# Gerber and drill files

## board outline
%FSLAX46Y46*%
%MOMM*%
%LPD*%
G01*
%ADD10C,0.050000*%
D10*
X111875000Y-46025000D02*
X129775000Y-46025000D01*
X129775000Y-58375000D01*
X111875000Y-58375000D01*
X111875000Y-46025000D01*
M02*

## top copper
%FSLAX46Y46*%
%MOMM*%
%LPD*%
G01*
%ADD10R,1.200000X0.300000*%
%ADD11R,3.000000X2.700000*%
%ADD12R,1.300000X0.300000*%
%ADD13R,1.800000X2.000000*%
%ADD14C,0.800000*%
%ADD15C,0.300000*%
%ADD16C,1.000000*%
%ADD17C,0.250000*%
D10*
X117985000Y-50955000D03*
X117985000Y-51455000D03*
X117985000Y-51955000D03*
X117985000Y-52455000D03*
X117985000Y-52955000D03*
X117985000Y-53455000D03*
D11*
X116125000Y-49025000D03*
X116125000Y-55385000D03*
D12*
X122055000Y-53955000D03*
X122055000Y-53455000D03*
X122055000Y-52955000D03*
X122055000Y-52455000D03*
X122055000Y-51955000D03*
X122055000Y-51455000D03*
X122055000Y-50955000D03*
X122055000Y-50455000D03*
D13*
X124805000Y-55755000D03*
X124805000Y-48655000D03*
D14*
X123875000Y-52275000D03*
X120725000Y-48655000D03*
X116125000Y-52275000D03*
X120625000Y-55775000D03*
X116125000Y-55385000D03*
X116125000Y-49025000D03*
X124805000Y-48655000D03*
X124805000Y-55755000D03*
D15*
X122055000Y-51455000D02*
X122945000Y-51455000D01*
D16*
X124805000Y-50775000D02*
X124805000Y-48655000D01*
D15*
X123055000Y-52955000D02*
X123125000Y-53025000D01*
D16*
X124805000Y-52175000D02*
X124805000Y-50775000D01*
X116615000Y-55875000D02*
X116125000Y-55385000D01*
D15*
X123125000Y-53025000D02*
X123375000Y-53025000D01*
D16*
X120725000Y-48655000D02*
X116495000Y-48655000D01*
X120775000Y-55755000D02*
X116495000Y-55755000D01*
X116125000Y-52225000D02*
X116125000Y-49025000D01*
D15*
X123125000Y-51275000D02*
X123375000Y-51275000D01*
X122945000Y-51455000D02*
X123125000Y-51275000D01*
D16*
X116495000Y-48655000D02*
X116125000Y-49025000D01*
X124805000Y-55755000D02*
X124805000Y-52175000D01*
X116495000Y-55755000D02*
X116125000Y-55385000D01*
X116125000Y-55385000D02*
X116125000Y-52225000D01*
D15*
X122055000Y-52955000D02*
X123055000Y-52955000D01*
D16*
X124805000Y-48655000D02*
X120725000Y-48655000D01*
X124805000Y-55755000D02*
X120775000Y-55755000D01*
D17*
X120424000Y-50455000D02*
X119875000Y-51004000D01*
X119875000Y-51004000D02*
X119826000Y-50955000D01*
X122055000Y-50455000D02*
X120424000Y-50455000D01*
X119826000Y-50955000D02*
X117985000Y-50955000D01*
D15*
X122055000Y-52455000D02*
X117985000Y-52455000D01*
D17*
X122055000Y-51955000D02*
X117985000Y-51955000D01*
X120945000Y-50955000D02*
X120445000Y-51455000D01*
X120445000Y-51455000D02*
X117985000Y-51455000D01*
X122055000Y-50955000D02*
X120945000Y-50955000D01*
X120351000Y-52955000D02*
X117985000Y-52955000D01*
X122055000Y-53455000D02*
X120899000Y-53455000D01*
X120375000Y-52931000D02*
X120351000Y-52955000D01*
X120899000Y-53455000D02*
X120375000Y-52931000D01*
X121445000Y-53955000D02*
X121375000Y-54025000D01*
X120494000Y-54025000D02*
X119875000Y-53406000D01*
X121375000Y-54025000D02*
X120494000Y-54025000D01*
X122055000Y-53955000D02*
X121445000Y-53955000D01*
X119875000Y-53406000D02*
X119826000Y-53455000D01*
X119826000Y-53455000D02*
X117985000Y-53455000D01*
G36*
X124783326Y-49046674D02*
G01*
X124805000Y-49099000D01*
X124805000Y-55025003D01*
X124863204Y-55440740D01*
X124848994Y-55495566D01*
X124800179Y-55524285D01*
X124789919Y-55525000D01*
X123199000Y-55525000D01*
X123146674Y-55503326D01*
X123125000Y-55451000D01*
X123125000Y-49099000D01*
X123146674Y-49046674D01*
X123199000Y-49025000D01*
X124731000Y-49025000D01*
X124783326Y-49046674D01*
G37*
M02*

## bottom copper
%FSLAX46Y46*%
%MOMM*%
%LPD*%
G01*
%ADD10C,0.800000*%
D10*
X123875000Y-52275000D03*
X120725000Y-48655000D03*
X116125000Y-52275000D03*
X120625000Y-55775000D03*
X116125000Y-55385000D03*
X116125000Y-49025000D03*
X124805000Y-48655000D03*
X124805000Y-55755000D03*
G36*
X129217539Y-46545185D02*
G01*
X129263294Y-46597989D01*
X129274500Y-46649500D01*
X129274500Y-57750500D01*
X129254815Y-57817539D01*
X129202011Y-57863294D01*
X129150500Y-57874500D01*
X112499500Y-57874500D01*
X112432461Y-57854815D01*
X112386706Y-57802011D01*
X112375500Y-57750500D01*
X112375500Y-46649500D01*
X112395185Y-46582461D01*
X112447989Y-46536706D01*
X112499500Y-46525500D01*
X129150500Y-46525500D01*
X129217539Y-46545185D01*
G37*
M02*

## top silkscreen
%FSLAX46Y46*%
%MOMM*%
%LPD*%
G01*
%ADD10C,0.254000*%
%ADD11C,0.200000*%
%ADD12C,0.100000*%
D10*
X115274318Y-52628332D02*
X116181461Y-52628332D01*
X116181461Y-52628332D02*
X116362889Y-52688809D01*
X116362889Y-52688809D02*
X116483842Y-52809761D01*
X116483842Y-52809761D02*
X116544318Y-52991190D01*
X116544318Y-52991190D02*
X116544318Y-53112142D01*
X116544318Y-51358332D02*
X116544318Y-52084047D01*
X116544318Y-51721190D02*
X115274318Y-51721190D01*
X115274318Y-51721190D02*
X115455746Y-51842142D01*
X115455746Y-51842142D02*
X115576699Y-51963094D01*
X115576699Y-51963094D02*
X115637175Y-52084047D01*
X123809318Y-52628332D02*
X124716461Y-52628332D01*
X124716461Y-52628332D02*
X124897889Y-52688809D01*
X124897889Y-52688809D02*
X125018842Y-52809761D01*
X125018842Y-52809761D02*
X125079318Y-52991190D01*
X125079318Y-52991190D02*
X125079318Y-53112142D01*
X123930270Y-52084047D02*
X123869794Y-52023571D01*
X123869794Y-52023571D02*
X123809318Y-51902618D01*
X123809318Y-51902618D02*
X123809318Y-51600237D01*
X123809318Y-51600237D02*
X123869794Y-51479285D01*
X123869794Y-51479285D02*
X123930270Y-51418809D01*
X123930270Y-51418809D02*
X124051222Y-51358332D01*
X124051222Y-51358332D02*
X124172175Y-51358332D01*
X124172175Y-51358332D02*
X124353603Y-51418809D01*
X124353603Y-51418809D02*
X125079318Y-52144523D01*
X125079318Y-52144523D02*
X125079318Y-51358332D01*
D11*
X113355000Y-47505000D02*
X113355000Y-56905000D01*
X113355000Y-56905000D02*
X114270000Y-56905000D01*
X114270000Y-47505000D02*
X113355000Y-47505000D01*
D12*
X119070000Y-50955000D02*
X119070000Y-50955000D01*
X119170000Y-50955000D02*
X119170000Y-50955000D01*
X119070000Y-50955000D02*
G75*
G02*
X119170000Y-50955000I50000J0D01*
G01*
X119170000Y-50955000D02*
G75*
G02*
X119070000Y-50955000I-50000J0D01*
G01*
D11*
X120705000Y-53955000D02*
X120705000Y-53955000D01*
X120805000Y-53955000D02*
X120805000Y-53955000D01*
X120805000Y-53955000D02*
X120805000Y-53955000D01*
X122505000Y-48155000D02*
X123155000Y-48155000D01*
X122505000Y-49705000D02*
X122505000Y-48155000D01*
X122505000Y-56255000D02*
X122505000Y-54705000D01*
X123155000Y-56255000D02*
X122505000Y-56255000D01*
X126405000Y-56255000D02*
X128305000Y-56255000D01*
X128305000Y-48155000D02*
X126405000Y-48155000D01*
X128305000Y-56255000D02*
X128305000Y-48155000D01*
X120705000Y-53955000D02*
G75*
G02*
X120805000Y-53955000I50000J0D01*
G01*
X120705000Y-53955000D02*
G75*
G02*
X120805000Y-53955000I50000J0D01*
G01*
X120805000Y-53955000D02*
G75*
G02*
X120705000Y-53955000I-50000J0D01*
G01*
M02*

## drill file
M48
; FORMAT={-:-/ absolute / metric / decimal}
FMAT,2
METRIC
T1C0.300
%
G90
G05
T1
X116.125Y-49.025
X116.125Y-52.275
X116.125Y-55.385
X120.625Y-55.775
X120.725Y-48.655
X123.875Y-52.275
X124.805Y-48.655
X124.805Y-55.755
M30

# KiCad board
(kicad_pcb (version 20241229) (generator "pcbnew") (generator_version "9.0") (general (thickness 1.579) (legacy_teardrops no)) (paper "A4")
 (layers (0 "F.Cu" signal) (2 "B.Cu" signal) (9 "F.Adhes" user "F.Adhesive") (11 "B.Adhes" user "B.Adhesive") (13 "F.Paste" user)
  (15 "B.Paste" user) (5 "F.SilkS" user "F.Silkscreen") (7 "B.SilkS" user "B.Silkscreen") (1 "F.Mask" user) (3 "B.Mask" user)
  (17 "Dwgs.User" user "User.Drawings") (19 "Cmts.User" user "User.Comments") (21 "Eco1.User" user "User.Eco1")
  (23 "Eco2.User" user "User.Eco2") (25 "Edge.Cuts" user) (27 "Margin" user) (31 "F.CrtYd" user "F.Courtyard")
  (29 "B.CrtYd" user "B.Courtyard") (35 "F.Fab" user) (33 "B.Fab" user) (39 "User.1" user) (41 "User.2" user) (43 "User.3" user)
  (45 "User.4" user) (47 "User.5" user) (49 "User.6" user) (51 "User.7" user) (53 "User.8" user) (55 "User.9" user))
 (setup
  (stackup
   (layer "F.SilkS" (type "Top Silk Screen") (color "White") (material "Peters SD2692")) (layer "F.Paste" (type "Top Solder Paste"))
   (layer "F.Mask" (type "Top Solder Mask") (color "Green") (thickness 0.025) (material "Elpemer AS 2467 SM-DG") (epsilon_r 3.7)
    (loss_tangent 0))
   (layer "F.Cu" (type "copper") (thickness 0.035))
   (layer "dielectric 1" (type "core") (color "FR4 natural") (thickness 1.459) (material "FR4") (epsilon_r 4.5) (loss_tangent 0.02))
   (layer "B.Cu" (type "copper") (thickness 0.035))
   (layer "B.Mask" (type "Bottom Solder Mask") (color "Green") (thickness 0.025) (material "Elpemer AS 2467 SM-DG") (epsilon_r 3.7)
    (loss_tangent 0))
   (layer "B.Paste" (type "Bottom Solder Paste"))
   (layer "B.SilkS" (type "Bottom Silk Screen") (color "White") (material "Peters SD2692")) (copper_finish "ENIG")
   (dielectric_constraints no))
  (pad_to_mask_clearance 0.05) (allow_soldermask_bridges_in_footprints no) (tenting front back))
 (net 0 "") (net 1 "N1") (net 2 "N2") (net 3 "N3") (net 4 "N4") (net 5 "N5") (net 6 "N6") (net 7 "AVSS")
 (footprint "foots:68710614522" (layer "F.Cu") (at 115.97 52.205 -90)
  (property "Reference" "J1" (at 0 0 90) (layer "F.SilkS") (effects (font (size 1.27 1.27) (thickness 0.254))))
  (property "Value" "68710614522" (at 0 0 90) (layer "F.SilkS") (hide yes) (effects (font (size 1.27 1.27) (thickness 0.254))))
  (fp_line (start -4.7 2.615) (end 4.7 2.615) (stroke (width 0.2) (type solid)) (layer "F.SilkS"))
  (fp_line (start 4.7 2.615) (end 4.7 1.7) (stroke (width 0.2) (type solid)) (layer "F.SilkS"))
  (fp_line (start -4.7 1.7) (end -4.7 2.615) (stroke (width 0.2) (type solid)) (layer "F.SilkS"))
  (fp_line (start -1.25 -3.1) (end -1.25 -3.1) (stroke (width 0.1) (type solid)) (layer "F.SilkS"))
  (fp_line (start -1.25 -3.2) (end -1.25 -3.2) (stroke (width 0.1) (type solid)) (layer "F.SilkS"))
  (fp_arc (start -1.25 -3.1) (mid -1.3 -3.15) (end -1.25 -3.2) (stroke (width 0.1) (type solid)) (layer "F.SilkS"))
  (fp_arc (start -1.25 -3.2) (mid -1.2 -3.15) (end -1.25 -3.1) (stroke (width 0.1) (type solid)) (layer "F.SilkS"))
  (pad "1" smd rect (at -1.25 -2.015 270) (size 0.3 1.2) (layers "F.Cu" "F.Mask" "F.Paste") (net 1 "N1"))
  (pad "2" smd rect (at -0.75 -2.015 270) (size 0.3 1.2) (layers "F.Cu" "F.Mask" "F.Paste") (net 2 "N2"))
  (pad "3" smd rect (at -0.25 -2.015 270) (size 0.3 1.2) (layers "F.Cu" "F.Mask" "F.Paste") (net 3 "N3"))
  (pad "4" smd rect (at 0.25 -2.015 270) (size 0.3 1.2) (layers "F.Cu" "F.Mask" "F.Paste") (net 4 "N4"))
  (pad "5" smd rect (at 0.75 -2.015 270) (size 0.3 1.2) (layers "F.Cu" "F.Mask" "F.Paste") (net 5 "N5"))
  (pad "6" smd rect (at 1.25 -2.015 270) (size 0.3 1.2) (layers "F.Cu" "F.Mask" "F.Paste") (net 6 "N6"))
  (pad "7" smd rect (at -3.18 -0.155 270) (size 2.7 3) (layers "F.Cu" "F.Mask" "F.Paste") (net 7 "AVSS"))
  (pad "8" smd rect (at 3.18 -0.155 270) (size 2.7 3) (layers "F.Cu" "F.Mask" "F.Paste") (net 7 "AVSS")))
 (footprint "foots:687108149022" (layer "F.Cu") (at 124.805 52.205 90)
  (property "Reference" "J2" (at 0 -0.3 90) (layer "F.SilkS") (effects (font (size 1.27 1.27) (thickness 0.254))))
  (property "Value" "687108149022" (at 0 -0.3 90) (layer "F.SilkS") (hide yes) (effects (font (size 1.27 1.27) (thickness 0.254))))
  (fp_line (start -1.75 -4.1) (end -1.75 -4.1) (stroke (width 0.2) (type solid)) (layer "F.SilkS"))
  (fp_line (start -1.75 -4) (end -1.75 -4) (stroke (width 0.2) (type solid)) (layer "F.SilkS"))
  (fp_line (start -1.75 -4) (end -1.75 -4) (stroke (width 0.2) (type solid)) (layer "F.SilkS"))
  (fp_line (start 4.05 -2.3) (end 4.05 -1.65) (stroke (width 0.2) (type solid)) (layer "F.SilkS"))
  (fp_line (start 2.5 -2.3) (end 4.05 -2.3) (stroke (width 0.2) (type solid)) (layer "F.SilkS"))
  (fp_line (start -4.05 -2.3) (end -2.5 -2.3) (stroke (width 0.2) (type solid)) (layer "F.SilkS"))
  (fp_line (start -4.05 -1.65) (end -4.05 -2.3) (stroke (width 0.2) (type solid)) (layer "F.SilkS"))
  (fp_line (start -4.05 1.6) (end -4.05 3.5) (stroke (width 0.2) (type solid)) (layer "F.SilkS"))
  (fp_line (start 4.05 3.5) (end 4.05 1.6) (stroke (width 0.2) (type solid)) (layer "F.SilkS"))
  (fp_line (start -4.05 3.5) (end 4.05 3.5) (stroke (width 0.2) (type solid)) (layer "F.SilkS"))
  (fp_arc (start -1.75 -4.1) (mid -1.7 -4.05) (end -1.75 -4) (stroke (width 0.2) (type solid)) (layer "F.SilkS"))
  (fp_arc (start -1.75 -4.1) (mid -1.7 -4.05) (end -1.75 -4) (stroke (width 0.2) (type solid)) (layer "F.SilkS"))
  (fp_arc (start -1.75 -4) (mid -1.8 -4.05) (end -1.75 -4.1) (stroke (width 0.2) (type solid)) (layer "F.SilkS"))
  (pad "1" smd rect (at -1.75 -2.75 90) (size 0.3 1.3) (layers "F.Cu" "F.Mask" "F.Paste") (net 6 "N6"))
  (pad "2" smd rect (at -1.25 -2.75 90) (size 0.3 1.3) (layers "F.Cu" "F.Mask" "F.Paste") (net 5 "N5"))
  (pad "3" smd rect (at -0.75 -2.75 90) (size 0.3 1.3) (layers "F.Cu" "F.Mask" "F.Paste") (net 7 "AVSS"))
  (pad "4" smd rect (at -0.25 -2.75 90) (size 0.3 1.3) (layers "F.Cu" "F.Mask" "F.Paste") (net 4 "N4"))
  (pad "5" smd rect (at 0.25 -2.75 90) (size 0.3 1.3) (layers "F.Cu" "F.Mask" "F.Paste") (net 3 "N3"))
  (pad "6" smd rect (at 0.75 -2.75 90) (size 0.3 1.3) (layers "F.Cu" "F.Mask" "F.Paste") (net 7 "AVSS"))
  (pad "7" smd rect (at 1.25 -2.75 90) (size 0.3 1.3) (layers "F.Cu" "F.Mask" "F.Paste") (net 2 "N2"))
  (pad "8" smd rect (at 1.75 -2.75 90) (size 0.3 1.3) (layers "F.Cu" "F.Mask" "F.Paste") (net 1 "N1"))
  (pad "MP1" smd rect (at -3.55 0 180) (size 1.8 2) (layers "F.Cu" "F.Mask" "F.Paste") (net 7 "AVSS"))
  (pad "MP2" smd rect (at 3.55 0 180) (size 1.8 2) (layers "F.Cu" "F.Mask" "F.Paste") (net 7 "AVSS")))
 (gr_rect (start 111.875 46.025) (end 129.775 58.375) (stroke (width 0.05) (type default)) (fill no) (layer "Edge.Cuts"))
 (segment (start 122.055 51.455) (end 122.945 51.455) (width 0.3) (layer "F.Cu") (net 7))
 (segment (start 124.805 50.775) (end 124.805 48.655) (width 1) (layer "F.Cu") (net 7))
 (segment (start 123.055 52.955) (end 123.125 53.025) (width 0.3) (layer "F.Cu") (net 7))
 (segment (start 124.805 52.175) (end 124.805 50.775) (width 1) (layer "F.Cu") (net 7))
 (segment (start 116.615 55.875) (end 116.125 55.385) (width 1) (layer "F.Cu") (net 7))
 (segment (start 123.125 53.025) (end 123.375 53.025) (width 0.3) (layer "F.Cu") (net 7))
 (segment (start 120.725 48.655) (end 116.495 48.655) (width 1) (layer "F.Cu") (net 7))
 (segment (start 120.775 55.755) (end 116.495 55.755) (width 1) (layer "F.Cu") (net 7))
 (segment (start 116.125 52.225) (end 116.125 49.025) (width 1) (layer "F.Cu") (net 7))
 (segment (start 123.125 51.275) (end 123.375 51.275) (width 0.3) (layer "F.Cu") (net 7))
 (segment (start 122.945 51.455) (end 123.125 51.275) (width 0.3) (layer "F.Cu") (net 7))
 (segment (start 116.495 48.655) (end 116.125 49.025) (width 1) (layer "F.Cu") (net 7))
 (segment (start 124.805 55.755) (end 124.805 52.175) (width 1) (layer "F.Cu") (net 7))
 (segment (start 116.495 55.755) (end 116.125 55.385) (width 1) (layer "F.Cu") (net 7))
 (segment (start 116.125 55.385) (end 116.125 52.225) (width 1) (layer "F.Cu") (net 7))
 (segment (start 122.055 52.955) (end 123.055 52.955) (width 0.3) (layer "F.Cu") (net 7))
 (segment (start 124.805 48.655) (end 120.725 48.655) (width 1) (layer "F.Cu") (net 7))
 (segment (start 124.805 55.755) (end 120.775 55.755) (width 1) (layer "F.Cu") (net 7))
 (via (at 123.875 52.275) (size 0.8) (drill 0.3) (layers "F.Cu" "B.Cu") (free yes) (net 7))
 (via (at 120.725 48.655) (size 0.8) (drill 0.3) (layers "F.Cu" "B.Cu") (free yes) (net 7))
 (via (at 116.125 52.275) (size 0.8) (drill 0.3) (layers "F.Cu" "B.Cu") (free yes) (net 7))
 (via (at 120.625 55.775) (size 0.8) (drill 0.3) (layers "F.Cu" "B.Cu") (free yes) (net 7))
 (via (at 116.125 55.385) (size 0.8) (drill 0.3) (layers "F.Cu" "B.Cu") (free yes) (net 7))
 (via (at 116.125 49.025) (size 0.8) (drill 0.3) (layers "F.Cu" "B.Cu") (free yes) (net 7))
 (via (at 124.805 48.655) (size 0.8) (drill 0.3) (layers "F.Cu" "B.Cu") (free yes) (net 7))
 (via (at 124.805 55.755) (size 0.8) (drill 0.3) (layers "F.Cu" "B.Cu") (free yes) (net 7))
 (segment (start 120.424 50.455) (end 119.875 51.004) (width 0.25) (layer "F.Cu") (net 1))
 (segment (start 119.875 51.004) (end 119.826 50.955) (width 0.25) (layer "F.Cu") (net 1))
 (segment (start 122.055 50.455) (end 120.424 50.455) (width 0.25) (layer "F.Cu") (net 1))
 (segment (start 119.826 50.955) (end 117.985 50.955) (width 0.25) (layer "F.Cu") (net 1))
 (segment (start 122.055 52.455) (end 117.985 52.455) (width 0.3) (layer "F.Cu") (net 4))
 (segment (start 122.055 51.955) (end 117.985 51.955) (width 0.25) (layer "F.Cu") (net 3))
 (segment (start 120.945 50.955) (end 120.445 51.455) (width 0.25) (layer "F.Cu") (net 2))
 (segment (start 120.445 51.455) (end 117.985 51.455) (width 0.25) (layer "F.Cu") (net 2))
 (segment (start 122.055 50.955) (end 120.945 50.955) (width 0.25) (layer "F.Cu") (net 2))
 (segment (start 120.351 52.955) (end 117.985 52.955) (width 0.25) (layer "F.Cu") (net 5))
 (segment (start 122.055 53.455) (end 120.899 53.455) (width 0.25) (layer "F.Cu") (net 5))
 (segment (start 120.375 52.931) (end 120.351 52.955) (width 0.25) (layer "F.Cu") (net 5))
 (segment (start 120.899 53.455) (end 120.375 52.931) (width 0.25) (layer "F.Cu") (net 5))
 (segment (start 121.445 53.955) (end 121.375 54.025) (width 0.25) (layer "F.Cu") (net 6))
 (segment (start 120.494 54.025) (end 119.875 53.406) (width 0.25) (layer "F.Cu") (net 6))
 (segment (start 121.375 54.025) (end 120.494 54.025) (width 0.25) (layer "F.Cu") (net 6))
 (segment (start 122.055 53.955) (end 121.445 53.955) (width 0.25) (layer "F.Cu") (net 6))
 (segment (start 119.875 53.406) (end 119.826 53.455) (width 0.25) (layer "F.Cu") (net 6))
 (segment (start 119.826 53.455) (end 117.985 53.455) (width 0.25) (layer "F.Cu") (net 6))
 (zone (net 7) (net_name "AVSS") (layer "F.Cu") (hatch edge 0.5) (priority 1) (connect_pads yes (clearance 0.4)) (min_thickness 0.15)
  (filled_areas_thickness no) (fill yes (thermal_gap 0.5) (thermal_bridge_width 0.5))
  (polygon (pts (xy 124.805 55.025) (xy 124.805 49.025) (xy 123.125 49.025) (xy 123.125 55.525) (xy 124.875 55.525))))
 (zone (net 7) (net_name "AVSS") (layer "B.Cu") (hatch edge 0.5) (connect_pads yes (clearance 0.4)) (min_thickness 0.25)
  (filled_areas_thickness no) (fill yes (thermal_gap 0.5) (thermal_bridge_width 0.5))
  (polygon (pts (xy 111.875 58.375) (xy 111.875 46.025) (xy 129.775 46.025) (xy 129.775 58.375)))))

